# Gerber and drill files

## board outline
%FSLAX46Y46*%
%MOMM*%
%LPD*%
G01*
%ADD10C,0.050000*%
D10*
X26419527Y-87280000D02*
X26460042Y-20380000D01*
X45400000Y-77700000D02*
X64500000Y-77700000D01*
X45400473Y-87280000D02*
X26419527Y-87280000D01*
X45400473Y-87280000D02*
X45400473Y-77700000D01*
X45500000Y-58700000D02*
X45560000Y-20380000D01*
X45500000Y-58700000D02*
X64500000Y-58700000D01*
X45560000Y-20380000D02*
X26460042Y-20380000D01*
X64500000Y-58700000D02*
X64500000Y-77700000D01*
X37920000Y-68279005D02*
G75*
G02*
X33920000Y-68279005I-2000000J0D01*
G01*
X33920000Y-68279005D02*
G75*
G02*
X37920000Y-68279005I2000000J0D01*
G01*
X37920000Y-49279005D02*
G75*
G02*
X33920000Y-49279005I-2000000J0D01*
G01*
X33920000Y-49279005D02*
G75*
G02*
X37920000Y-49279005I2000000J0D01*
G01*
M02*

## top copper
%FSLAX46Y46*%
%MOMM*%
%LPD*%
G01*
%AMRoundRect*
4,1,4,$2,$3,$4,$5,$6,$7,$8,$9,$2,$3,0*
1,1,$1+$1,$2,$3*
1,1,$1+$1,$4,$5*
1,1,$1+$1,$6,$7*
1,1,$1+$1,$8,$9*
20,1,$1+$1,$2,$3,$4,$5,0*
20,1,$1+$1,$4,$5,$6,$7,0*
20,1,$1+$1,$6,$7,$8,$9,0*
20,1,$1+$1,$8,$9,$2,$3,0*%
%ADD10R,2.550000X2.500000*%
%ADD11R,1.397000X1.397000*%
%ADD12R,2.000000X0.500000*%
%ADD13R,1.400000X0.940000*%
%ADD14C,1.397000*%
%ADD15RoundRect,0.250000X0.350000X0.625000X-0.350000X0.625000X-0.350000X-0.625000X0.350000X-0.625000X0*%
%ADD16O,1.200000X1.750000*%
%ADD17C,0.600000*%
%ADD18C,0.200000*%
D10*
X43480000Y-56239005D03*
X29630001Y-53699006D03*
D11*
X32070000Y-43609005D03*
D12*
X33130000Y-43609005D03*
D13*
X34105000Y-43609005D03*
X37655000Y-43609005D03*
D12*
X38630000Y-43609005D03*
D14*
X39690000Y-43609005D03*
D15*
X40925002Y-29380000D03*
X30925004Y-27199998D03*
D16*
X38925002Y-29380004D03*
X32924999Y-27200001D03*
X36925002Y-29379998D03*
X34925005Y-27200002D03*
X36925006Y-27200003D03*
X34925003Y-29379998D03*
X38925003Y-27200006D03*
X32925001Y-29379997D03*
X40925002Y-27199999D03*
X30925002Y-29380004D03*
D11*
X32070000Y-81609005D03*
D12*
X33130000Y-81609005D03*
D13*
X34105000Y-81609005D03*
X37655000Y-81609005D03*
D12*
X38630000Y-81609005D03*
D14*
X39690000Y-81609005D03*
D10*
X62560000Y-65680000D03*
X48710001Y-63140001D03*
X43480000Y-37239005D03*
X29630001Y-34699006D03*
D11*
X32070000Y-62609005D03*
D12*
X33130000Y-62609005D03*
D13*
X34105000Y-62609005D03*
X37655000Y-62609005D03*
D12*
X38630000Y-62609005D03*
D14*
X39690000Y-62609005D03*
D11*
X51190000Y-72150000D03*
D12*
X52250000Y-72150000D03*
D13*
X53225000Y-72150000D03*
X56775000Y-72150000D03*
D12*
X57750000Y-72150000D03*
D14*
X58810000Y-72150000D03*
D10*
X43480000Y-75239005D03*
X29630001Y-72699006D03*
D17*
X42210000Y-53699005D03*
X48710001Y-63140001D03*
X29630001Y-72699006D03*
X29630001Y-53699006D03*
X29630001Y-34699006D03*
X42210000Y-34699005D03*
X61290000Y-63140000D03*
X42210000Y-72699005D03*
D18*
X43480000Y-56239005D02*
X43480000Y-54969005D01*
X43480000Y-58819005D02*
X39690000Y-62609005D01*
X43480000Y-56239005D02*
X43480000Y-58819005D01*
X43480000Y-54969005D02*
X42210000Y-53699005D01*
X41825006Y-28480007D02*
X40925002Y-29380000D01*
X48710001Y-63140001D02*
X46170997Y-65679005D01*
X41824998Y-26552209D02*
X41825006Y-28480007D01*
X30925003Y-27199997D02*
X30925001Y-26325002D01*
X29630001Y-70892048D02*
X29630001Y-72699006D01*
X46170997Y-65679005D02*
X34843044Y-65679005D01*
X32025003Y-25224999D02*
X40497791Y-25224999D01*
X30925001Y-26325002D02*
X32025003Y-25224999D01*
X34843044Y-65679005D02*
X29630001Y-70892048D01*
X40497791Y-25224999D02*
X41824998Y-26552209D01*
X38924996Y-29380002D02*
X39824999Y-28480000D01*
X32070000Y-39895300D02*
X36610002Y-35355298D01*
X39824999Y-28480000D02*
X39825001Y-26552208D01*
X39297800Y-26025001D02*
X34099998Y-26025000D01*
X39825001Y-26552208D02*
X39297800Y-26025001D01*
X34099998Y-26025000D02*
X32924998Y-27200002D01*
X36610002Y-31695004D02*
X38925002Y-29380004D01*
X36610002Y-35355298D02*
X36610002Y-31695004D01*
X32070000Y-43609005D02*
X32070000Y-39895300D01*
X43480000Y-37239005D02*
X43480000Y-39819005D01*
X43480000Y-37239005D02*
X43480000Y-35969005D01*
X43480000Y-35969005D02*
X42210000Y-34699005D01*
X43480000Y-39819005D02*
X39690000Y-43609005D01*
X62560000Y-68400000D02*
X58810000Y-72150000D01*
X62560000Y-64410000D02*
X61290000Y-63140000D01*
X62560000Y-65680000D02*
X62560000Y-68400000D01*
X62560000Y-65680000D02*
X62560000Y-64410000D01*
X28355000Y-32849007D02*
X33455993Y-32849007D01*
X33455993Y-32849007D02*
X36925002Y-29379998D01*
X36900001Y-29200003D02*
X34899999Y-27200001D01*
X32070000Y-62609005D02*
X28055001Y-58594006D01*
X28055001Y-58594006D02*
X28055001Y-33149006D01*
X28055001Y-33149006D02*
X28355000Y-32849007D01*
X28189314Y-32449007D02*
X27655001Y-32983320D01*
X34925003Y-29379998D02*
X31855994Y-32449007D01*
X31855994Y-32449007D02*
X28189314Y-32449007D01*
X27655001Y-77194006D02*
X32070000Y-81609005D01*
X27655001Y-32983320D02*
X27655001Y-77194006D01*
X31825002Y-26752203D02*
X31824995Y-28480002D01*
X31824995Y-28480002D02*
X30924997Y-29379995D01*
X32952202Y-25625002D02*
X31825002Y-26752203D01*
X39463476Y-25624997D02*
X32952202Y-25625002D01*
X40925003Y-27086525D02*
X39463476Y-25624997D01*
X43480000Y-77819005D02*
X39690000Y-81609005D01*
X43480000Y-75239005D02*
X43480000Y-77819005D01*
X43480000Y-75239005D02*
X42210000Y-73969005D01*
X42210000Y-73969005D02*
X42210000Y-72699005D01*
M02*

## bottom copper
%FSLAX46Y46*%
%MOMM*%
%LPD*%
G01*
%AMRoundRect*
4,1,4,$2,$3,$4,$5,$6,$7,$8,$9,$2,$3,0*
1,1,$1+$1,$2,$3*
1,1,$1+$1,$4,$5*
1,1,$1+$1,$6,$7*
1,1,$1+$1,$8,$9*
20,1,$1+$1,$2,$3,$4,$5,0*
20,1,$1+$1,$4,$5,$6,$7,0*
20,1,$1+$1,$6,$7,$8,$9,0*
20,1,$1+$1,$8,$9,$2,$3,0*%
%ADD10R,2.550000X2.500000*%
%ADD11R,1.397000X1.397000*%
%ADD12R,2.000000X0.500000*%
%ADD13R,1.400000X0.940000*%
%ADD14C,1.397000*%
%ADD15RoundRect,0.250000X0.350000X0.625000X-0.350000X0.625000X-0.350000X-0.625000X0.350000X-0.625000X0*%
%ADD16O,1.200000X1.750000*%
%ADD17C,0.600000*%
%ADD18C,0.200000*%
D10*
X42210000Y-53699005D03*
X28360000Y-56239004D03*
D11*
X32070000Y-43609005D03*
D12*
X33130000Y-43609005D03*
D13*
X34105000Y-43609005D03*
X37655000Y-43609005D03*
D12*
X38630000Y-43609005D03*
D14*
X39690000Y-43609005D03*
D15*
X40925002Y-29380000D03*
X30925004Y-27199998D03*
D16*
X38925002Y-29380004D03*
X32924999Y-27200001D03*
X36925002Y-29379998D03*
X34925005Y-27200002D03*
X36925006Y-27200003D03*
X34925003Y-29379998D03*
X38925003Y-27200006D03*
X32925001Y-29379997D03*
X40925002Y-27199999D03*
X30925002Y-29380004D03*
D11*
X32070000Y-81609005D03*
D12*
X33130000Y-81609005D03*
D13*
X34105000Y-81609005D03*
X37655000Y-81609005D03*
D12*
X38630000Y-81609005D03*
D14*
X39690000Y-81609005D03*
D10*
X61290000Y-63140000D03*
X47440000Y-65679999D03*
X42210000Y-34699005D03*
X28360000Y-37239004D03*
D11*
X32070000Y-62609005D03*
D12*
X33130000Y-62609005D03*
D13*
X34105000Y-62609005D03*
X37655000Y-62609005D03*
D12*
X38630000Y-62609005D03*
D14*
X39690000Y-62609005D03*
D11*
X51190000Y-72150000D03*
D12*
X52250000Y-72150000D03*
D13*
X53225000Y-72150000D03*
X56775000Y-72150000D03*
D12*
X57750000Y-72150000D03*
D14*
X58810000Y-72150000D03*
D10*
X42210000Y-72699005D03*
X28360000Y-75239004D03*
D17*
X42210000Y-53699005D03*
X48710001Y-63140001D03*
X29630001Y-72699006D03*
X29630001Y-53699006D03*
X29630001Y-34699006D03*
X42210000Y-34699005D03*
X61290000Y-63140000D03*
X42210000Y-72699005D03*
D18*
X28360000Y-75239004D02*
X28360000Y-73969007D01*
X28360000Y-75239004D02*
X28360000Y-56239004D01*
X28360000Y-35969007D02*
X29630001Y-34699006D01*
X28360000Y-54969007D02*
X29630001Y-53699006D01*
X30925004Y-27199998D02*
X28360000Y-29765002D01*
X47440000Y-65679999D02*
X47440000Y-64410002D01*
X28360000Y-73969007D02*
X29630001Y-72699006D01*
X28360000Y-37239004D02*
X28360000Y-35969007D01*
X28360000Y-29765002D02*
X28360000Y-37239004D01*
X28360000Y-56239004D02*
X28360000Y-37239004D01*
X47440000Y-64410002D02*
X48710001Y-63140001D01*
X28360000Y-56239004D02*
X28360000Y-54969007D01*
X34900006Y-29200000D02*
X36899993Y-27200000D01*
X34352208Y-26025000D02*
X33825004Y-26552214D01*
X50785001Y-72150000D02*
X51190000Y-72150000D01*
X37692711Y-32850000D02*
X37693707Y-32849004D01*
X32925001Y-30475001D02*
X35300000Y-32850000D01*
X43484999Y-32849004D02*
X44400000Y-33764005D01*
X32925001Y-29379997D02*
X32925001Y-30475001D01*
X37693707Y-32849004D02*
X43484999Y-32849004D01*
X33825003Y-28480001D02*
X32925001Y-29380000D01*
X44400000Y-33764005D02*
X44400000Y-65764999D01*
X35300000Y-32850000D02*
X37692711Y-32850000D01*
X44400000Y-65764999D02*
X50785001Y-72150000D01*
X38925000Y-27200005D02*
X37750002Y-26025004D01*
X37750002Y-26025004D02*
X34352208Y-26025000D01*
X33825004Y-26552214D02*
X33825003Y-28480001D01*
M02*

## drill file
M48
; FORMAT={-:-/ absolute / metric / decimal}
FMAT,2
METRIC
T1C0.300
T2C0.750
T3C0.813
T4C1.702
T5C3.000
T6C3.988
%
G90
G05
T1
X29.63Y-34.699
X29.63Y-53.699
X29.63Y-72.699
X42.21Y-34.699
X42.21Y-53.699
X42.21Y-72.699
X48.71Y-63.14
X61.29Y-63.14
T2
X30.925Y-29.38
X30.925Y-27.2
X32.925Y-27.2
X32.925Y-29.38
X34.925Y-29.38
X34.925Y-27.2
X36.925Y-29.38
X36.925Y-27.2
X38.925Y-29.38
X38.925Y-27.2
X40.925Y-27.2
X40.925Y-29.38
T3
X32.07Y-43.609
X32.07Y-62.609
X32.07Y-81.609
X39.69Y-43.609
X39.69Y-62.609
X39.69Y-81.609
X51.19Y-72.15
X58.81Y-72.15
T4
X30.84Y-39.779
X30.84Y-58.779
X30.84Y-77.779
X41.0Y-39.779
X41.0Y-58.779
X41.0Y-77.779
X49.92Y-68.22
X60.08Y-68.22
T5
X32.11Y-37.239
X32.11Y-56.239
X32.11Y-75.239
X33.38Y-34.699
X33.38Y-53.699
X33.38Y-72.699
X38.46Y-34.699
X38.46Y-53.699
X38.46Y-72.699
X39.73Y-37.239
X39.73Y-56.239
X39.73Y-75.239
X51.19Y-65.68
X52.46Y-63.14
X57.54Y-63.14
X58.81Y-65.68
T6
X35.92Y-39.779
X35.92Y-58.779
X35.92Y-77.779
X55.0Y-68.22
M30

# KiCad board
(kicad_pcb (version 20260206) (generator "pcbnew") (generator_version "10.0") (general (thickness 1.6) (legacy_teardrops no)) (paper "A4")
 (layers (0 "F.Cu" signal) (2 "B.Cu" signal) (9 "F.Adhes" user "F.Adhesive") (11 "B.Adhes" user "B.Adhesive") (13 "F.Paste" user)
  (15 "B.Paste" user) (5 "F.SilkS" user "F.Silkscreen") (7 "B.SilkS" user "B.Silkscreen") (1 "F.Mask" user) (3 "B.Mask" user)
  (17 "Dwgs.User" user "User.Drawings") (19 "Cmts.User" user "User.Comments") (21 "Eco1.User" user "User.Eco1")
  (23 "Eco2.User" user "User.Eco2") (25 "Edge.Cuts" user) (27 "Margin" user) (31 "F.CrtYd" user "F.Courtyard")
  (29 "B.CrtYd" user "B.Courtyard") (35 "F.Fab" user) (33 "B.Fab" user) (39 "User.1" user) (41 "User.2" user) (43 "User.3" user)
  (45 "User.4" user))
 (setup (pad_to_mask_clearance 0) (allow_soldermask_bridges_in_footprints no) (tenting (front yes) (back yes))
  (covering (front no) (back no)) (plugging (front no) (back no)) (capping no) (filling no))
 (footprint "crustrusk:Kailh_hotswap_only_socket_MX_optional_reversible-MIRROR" (layer "F.Cu") (at 35.92 58.779005)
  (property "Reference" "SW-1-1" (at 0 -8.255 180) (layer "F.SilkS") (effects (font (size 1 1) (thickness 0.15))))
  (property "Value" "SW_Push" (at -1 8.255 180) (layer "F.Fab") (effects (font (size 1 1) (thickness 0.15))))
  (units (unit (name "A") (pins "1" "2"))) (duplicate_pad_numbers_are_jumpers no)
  (pad "" np_thru_hole circle (at -5.08 0) (size 1.7018 1.7018) (drill 1.7018) (layers "*.Cu" "*.Mask"))
  (pad "" np_thru_hole circle (at -3.81 -2.54 180) (size 3 3) (drill 3) (layers "*.Cu" "*.Mask"))
  (pad "" np_thru_hole circle (at -2.54 -5.079998) (size 3 3) (drill 3) (layers "*.Cu" "*.Mask"))
  (pad "" np_thru_hole circle (at 0 0) (size 3.9878 3.9878) (drill 3.9878) (layers "*.Cu" "*.Mask"))
  (pad "" np_thru_hole circle (at 2.540002 -5.080001 180) (size 3 3) (drill 3) (layers "*.Cu" "*.Mask"))
  (pad "" np_thru_hole circle (at 3.81 -2.54) (size 3 3) (drill 3) (layers "*.Cu" "*.Mask"))
  (pad "" np_thru_hole circle (at 5.08 0) (size 1.7018 1.7018) (drill 1.7018) (layers "*.Cu" "*.Mask"))
  (pad "1" smd rect (at 6.29 -5.08 180) (size 2.55 2.5) (layers "B.Cu" "B.Mask" "B.Paste") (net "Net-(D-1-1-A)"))
  (pad "1" smd rect (at 7.56 -2.54) (size 2.55 2.5) (layers "F.Cu" "F.Mask" "F.Paste") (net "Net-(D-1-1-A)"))
  (pad "2" smd rect (at -7.56 -2.540001 180) (size 2.55 2.5) (layers "B.Cu" "B.Mask" "B.Paste") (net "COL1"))
  (pad "2" smd rect (at -6.289999 -5.079999) (size 2.55 2.5) (layers "F.Cu" "F.Mask" "F.Paste") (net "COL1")))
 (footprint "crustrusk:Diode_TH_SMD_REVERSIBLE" (layer "F.Cu") (at 35.88 43.609005)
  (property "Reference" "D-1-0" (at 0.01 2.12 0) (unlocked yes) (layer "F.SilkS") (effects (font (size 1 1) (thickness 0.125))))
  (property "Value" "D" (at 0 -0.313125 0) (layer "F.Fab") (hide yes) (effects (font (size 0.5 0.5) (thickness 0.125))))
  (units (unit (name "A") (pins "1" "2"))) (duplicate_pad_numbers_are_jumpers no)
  (pad "1" thru_hole rect (at -3.81 0) (size 1.397 1.397) (drill 0.8128) (layers "*.Cu" "*.Mask") (remove_unused_layers no) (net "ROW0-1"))
  (pad "1" smd rect (at -2.75 0 180) (size 2 0.5) (layers "F.Cu") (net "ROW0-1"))
  (pad "1" smd rect (at -2.75 0) (size 2 0.5) (layers "B.Cu") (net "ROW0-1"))
  (pad "1" smd rect (at -1.775 0 180) (size 1.4 0.94) (layers "F.Cu" "F.Mask" "F.Paste") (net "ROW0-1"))
  (pad "1" smd rect (at -1.775 0) (size 1.4 0.94) (layers "B.Cu" "B.Mask" "B.Paste") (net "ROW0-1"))
  (pad "2" smd rect (at 1.775 0 180) (size 1.4 0.94) (layers "F.Cu" "F.Mask" "F.Paste") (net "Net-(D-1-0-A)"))
  (pad "2" smd rect (at 1.775 0) (size 1.4 0.94) (layers "B.Cu" "B.Mask" "B.Paste") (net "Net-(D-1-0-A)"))
  (pad "2" smd rect (at 2.75 0 180) (size 2 0.5) (layers "F.Cu") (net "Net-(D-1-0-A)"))
  (pad "2" smd rect (at 2.75 0) (size 2 0.5) (layers "B.Cu") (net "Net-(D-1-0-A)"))
  (pad "2" thru_hole circle (at 3.81 0) (size 1.397 1.397) (drill 0.8128) (layers "*.Cu" "*.Mask") (remove_unused_layers no)
   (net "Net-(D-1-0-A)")))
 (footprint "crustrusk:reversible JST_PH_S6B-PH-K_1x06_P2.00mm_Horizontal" (layer "F.Cu") (at 40.925002 29.38 180)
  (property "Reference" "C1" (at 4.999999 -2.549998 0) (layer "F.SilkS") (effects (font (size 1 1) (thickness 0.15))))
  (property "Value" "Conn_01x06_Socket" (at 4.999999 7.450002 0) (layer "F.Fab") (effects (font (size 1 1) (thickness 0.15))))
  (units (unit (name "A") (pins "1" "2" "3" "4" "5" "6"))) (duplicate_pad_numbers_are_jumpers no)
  (pad "1" thru_hole roundrect (at 0 0 180) (size 1.2 1.75) (drill 0.75) (layers "*.Cu" "*.Mask") (remove_unused_layers no)
   (roundrect_rratio 0.208333) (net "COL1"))
  (pad "1" thru_hole roundrect (at 9.999998 2.180002 180) (size 1.2 1.75) (drill 0.75) (layers "*.Cu" "*.Mask") (remove_unused_layers no)
   (roundrect_rratio 0.208333) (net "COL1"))
  (pad "2" thru_hole oval (at 2 -0.000004 180) (size 1.2 1.75) (drill 0.75) (layers "*.Cu" "*.Mask") (remove_unused_layers no)
   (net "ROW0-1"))
  (pad "2" thru_hole oval (at 8.000003 2.179999 180) (size 1.2 1.75) (drill 0.75) (layers "*.Cu" "*.Mask") (remove_unused_layers no)
   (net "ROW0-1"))
  (pad "3" thru_hole oval (at 4 0.000002 180) (size 1.2 1.75) (drill 0.75) (layers "*.Cu" "*.Mask") (remove_unused_layers no) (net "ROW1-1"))
  (pad "3" thru_hole oval (at 5.999997 2.179998 180) (size 1.2 1.75) (drill 0.75) (layers "*.Cu" "*.Mask") (remove_unused_layers no)
   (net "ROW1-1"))
  (pad "4" thru_hole oval (at 3.999996 2.179997 180) (size 1.2 1.75) (drill 0.75) (layers "*.Cu" "*.Mask") (remove_unused_layers no)
   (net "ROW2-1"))
  (pad "4" thru_hole oval (at 5.999999 0.000002 180) (size 1.2 1.75) (drill 0.75) (layers "*.Cu" "*.Mask") (remove_unused_layers no)
   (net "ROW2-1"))
  (pad "5" thru_hole oval (at 1.999999 2.179994 180) (size 1.2 1.75) (drill 0.75) (layers "*.Cu" "*.Mask") (remove_unused_layers no)
   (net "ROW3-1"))
  (pad "5" thru_hole oval (at 8.000001 0.000003 180) (size 1.2 1.75) (drill 0.75) (layers "*.Cu" "*.Mask") (remove_unused_layers no)
   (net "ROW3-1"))
  (pad "6" thru_hole oval (at 0 2.180001 180) (size 1.2 1.75) (drill 0.75) (layers "*.Cu" "*.Mask") (remove_unused_layers no) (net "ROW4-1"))
  (pad "6" thru_hole oval (at 10 -0.000004 180) (size 1.2 1.75) (drill 0.75) (layers "*.Cu" "*.Mask") (remove_unused_layers no)
   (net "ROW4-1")))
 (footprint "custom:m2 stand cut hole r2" (layer "F.Cu") (at 35.92 68.279005)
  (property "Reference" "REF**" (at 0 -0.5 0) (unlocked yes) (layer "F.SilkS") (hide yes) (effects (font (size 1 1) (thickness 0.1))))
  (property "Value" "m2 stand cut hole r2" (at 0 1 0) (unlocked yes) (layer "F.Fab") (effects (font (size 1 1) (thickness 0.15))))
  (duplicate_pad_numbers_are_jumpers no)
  (fp_circle (center 0 0) (end 2 0) (stroke (width 0.05) (type default)) (fill no) (layer "Edge.Cuts")))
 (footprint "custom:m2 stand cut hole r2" (layer "F.Cu") (at 35.92 49.279005)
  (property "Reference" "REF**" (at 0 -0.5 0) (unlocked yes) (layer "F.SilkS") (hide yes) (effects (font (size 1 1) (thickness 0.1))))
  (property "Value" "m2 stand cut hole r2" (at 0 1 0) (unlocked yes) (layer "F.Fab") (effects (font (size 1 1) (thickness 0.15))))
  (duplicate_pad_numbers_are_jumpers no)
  (fp_circle (center 0 0) (end 2 0) (stroke (width 0.05) (type default)) (fill no) (layer "Edge.Cuts")))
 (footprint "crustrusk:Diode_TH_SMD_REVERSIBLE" (layer "F.Cu") (at 35.88 81.609005)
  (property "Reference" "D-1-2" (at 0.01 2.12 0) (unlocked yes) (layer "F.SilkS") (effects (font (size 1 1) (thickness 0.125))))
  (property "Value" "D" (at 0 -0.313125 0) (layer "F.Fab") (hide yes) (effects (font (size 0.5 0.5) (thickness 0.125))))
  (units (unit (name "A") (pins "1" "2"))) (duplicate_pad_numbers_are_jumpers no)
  (pad "1" thru_hole rect (at -3.81 0) (size 1.397 1.397) (drill 0.8128) (layers "*.Cu" "*.Mask") (remove_unused_layers no) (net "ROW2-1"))
  (pad "1" smd rect (at -2.75 0 180) (size 2 0.5) (layers "F.Cu") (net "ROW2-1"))
  (pad "1" smd rect (at -2.75 0) (size 2 0.5) (layers "B.Cu") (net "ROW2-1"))
  (pad "1" smd rect (at -1.775 0 180) (size 1.4 0.94) (layers "F.Cu" "F.Mask" "F.Paste") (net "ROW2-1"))
  (pad "1" smd rect (at -1.775 0) (size 1.4 0.94) (layers "B.Cu" "B.Mask" "B.Paste") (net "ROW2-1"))
  (pad "2" smd rect (at 1.775 0 180) (size 1.4 0.94) (layers "F.Cu" "F.Mask" "F.Paste") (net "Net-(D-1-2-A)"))
  (pad "2" smd rect (at 1.775 0) (size 1.4 0.94) (layers "B.Cu" "B.Mask" "B.Paste") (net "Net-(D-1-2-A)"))
  (pad "2" smd rect (at 2.75 0 180) (size 2 0.5) (layers "F.Cu") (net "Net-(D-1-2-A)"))
  (pad "2" smd rect (at 2.75 0) (size 2 0.5) (layers "B.Cu") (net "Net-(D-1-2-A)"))
  (pad "2" thru_hole circle (at 3.81 0) (size 1.397 1.397) (drill 0.8128) (layers "*.Cu" "*.Mask") (remove_unused_layers no)
   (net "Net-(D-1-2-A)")))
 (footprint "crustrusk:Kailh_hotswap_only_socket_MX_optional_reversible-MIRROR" (layer "F.Cu") (at 55 68.22)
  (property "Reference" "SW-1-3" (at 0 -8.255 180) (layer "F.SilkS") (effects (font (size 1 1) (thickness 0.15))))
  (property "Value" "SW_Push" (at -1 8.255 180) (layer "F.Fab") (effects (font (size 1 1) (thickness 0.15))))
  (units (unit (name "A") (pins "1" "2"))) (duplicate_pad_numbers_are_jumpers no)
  (pad "" np_thru_hole circle (at -5.08 0) (size 1.7018 1.7018) (drill 1.7018) (layers "*.Cu" "*.Mask"))
  (pad "" np_thru_hole circle (at -3.81 -2.54 180) (size 3 3) (drill 3) (layers "*.Cu" "*.Mask"))
  (pad "" np_thru_hole circle (at -2.54 -5.079998) (size 3 3) (drill 3) (layers "*.Cu" "*.Mask"))
  (pad "" np_thru_hole circle (at 0 0) (size 3.9878 3.9878) (drill 3.9878) (layers "*.Cu" "*.Mask"))
  (pad "" np_thru_hole circle (at 2.540002 -5.080001 180) (size 3 3) (drill 3) (layers "*.Cu" "*.Mask"))
  (pad "" np_thru_hole circle (at 3.81 -2.54) (size 3 3) (drill 3) (layers "*.Cu" "*.Mask"))
  (pad "" np_thru_hole circle (at 5.08 0) (size 1.7018 1.7018) (drill 1.7018) (layers "*.Cu" "*.Mask"))
  (pad "1" smd rect (at 6.29 -5.08 180) (size 2.55 2.5) (layers "B.Cu" "B.Mask" "B.Paste") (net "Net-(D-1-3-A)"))
  (pad "1" smd rect (at 7.56 -2.54) (size 2.55 2.5) (layers "F.Cu" "F.Mask" "F.Paste") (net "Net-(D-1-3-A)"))
  (pad "2" smd rect (at -7.56 -2.540001 180) (size 2.55 2.5) (layers "B.Cu" "B.Mask" "B.Paste") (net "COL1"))
  (pad "2" smd rect (at -6.289999 -5.079999) (size 2.55 2.5) (layers "F.Cu" "F.Mask" "F.Paste") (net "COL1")))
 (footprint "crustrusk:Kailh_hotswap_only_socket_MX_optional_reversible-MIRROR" (layer "F.Cu") (at 35.92 39.779005)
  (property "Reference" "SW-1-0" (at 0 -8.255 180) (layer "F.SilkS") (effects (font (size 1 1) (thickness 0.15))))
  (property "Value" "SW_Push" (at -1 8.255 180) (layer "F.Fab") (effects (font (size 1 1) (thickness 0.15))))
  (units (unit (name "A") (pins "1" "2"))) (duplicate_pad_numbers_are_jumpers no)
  (pad "" np_thru_hole circle (at -5.08 0) (size 1.7018 1.7018) (drill 1.7018) (layers "*.Cu" "*.Mask"))
  (pad "" np_thru_hole circle (at -3.81 -2.54 180) (size 3 3) (drill 3) (layers "*.Cu" "*.Mask"))
  (pad "" np_thru_hole circle (at -2.54 -5.079998) (size 3 3) (drill 3) (layers "*.Cu" "*.Mask"))
  (pad "" np_thru_hole circle (at 0 0) (size 3.9878 3.9878) (drill 3.9878) (layers "*.Cu" "*.Mask"))
  (pad "" np_thru_hole circle (at 2.540002 -5.080001 180) (size 3 3) (drill 3) (layers "*.Cu" "*.Mask"))
  (pad "" np_thru_hole circle (at 3.81 -2.54) (size 3 3) (drill 3) (layers "*.Cu" "*.Mask"))
  (pad "" np_thru_hole circle (at 5.08 0) (size 1.7018 1.7018) (drill 1.7018) (layers "*.Cu" "*.Mask"))
  (pad "1" smd rect (at 6.29 -5.08 180) (size 2.55 2.5) (layers "B.Cu" "B.Mask" "B.Paste") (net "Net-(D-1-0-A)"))
  (pad "1" smd rect (at 7.56 -2.54) (size 2.55 2.5) (layers "F.Cu" "F.Mask" "F.Paste") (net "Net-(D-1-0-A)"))
  (pad "2" smd rect (at -7.56 -2.540001 180) (size 2.55 2.5) (layers "B.Cu" "B.Mask" "B.Paste") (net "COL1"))
  (pad "2" smd rect (at -6.289999 -5.079999) (size 2.55 2.5) (layers "F.Cu" "F.Mask" "F.Paste") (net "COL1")))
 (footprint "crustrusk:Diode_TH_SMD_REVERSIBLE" (layer "F.Cu") (at 35.88 62.609005)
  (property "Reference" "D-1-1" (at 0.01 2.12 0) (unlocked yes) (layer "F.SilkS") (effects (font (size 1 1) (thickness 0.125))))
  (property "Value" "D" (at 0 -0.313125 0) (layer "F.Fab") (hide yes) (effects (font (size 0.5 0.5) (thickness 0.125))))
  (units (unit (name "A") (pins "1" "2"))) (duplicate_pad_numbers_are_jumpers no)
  (pad "1" thru_hole rect (at -3.81 0) (size 1.397 1.397) (drill 0.8128) (layers "*.Cu" "*.Mask") (remove_unused_layers no) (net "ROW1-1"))
  (pad "1" smd rect (at -2.75 0 180) (size 2 0.5) (layers "F.Cu") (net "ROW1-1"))
  (pad "1" smd rect (at -2.75 0) (size 2 0.5) (layers "B.Cu") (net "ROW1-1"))
  (pad "1" smd rect (at -1.775 0 180) (size 1.4 0.94) (layers "F.Cu" "F.Mask" "F.Paste") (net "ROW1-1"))
  (pad "1" smd rect (at -1.775 0) (size 1.4 0.94) (layers "B.Cu" "B.Mask" "B.Paste") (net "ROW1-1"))
  (pad "2" smd rect (at 1.775 0 180) (size 1.4 0.94) (layers "F.Cu" "F.Mask" "F.Paste") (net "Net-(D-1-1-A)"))
  (pad "2" smd rect (at 1.775 0) (size 1.4 0.94) (layers "B.Cu" "B.Mask" "B.Paste") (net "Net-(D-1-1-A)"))
  (pad "2" smd rect (at 2.75 0 180) (size 2 0.5) (layers "F.Cu") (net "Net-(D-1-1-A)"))
  (pad "2" smd rect (at 2.75 0) (size 2 0.5) (layers "B.Cu") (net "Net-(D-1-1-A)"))
  (pad "2" thru_hole circle (at 3.81 0) (size 1.397 1.397) (drill 0.8128) (layers "*.Cu" "*.Mask") (remove_unused_layers no)
   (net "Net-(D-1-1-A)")))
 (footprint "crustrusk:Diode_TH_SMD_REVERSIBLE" (layer "F.Cu") (at 55 72.15)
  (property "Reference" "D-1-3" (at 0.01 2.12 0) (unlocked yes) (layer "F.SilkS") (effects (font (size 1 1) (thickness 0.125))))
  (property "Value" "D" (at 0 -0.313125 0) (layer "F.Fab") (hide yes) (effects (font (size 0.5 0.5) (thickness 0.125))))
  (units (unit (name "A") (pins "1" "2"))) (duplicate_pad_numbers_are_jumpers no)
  (pad "1" thru_hole rect (at -3.81 0) (size 1.397 1.397) (drill 0.8128) (layers "*.Cu" "*.Mask") (remove_unused_layers no) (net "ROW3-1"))
  (pad "1" smd rect (at -2.75 0 180) (size 2 0.5) (layers "F.Cu") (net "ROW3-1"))
  (pad "1" smd rect (at -2.75 0) (size 2 0.5) (layers "B.Cu") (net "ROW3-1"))
  (pad "1" smd rect (at -1.775 0 180) (size 1.4 0.94) (layers "F.Cu" "F.Mask" "F.Paste") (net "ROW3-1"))
  (pad "1" smd rect (at -1.775 0) (size 1.4 0.94) (layers "B.Cu" "B.Mask" "B.Paste") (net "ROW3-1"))
  (pad "2" smd rect (at 1.775 0 180) (size 1.4 0.94) (layers "F.Cu" "F.Mask" "F.Paste") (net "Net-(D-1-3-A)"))
  (pad "2" smd rect (at 1.775 0) (size 1.4 0.94) (layers "B.Cu" "B.Mask" "B.Paste") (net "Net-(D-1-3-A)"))
  (pad "2" smd rect (at 2.75 0 180) (size 2 0.5) (layers "F.Cu") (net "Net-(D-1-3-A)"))
  (pad "2" smd rect (at 2.75 0) (size 2 0.5) (layers "B.Cu") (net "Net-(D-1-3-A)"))
  (pad "2" thru_hole circle (at 3.81 0) (size 1.397 1.397) (drill 0.8128) (layers "*.Cu" "*.Mask") (remove_unused_layers no)
   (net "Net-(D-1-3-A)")))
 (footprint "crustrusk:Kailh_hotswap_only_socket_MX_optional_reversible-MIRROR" (layer "F.Cu") (at 35.92 77.779005)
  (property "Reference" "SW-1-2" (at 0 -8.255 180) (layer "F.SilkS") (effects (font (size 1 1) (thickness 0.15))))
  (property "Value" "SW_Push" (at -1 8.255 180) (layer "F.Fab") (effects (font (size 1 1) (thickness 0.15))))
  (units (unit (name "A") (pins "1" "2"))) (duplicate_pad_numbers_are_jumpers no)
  (pad "" np_thru_hole circle (at -5.08 0) (size 1.7018 1.7018) (drill 1.7018) (layers "*.Cu" "*.Mask"))
  (pad "" np_thru_hole circle (at -3.81 -2.54 180) (size 3 3) (drill 3) (layers "*.Cu" "*.Mask"))
  (pad "" np_thru_hole circle (at -2.54 -5.079998) (size 3 3) (drill 3) (layers "*.Cu" "*.Mask"))
  (pad "" np_thru_hole circle (at 0 0) (size 3.9878 3.9878) (drill 3.9878) (layers "*.Cu" "*.Mask"))
  (pad "" np_thru_hole circle (at 2.540002 -5.080001 180) (size 3 3) (drill 3) (layers "*.Cu" "*.Mask"))
  (pad "" np_thru_hole circle (at 3.81 -2.54) (size 3 3) (drill 3) (layers "*.Cu" "*.Mask"))
  (pad "" np_thru_hole circle (at 5.08 0) (size 1.7018 1.7018) (drill 1.7018) (layers "*.Cu" "*.Mask"))
  (pad "1" smd rect (at 6.29 -5.08 180) (size 2.55 2.5) (layers "B.Cu" "B.Mask" "B.Paste") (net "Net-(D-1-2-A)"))
  (pad "1" smd rect (at 7.56 -2.54) (size 2.55 2.5) (layers "F.Cu" "F.Mask" "F.Paste") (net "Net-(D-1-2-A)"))
  (pad "2" smd rect (at -7.56 -2.540001 180) (size 2.55 2.5) (layers "B.Cu" "B.Mask" "B.Paste") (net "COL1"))
  (pad "2" smd rect (at -6.289999 -5.079999) (size 2.55 2.5) (layers "F.Cu" "F.Mask" "F.Paste") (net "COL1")))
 (gr_line (start 26.419527 87.28) (end 26.460042 20.38) (stroke (width 0.05) (type default)) (layer "Edge.Cuts"))
 (gr_line (start 45.4 77.7) (end 64.5 77.7) (stroke (width 0.05) (type default)) (layer "Edge.Cuts"))
 (gr_line (start 45.400473 87.28) (end 26.419527 87.28) (stroke (width 0.05) (type default)) (layer "Edge.Cuts"))
 (gr_line (start 45.400473 87.28) (end 45.400473 77.7) (stroke (width 0.05) (type default)) (layer "Edge.Cuts"))
 (gr_line (start 45.5 58.7) (end 45.56 20.38) (stroke (width 0.05) (type default)) (layer "Edge.Cuts"))
 (gr_line (start 45.5 58.7) (end 64.5 58.7) (stroke (width 0.05) (type default)) (layer "Edge.Cuts"))
 (gr_line (start 45.56 20.38) (end 26.460042 20.38) (stroke (width 0.05) (type default)) (layer "Edge.Cuts"))
 (gr_line (start 64.5 58.7) (end 64.5 77.7) (stroke (width 0.05) (type default)) (layer "Edge.Cuts"))
 (segment (start 43.48 56.239005) (end 43.48 54.969005) (width 0.2) (layer "F.Cu") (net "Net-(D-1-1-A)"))
 (segment (start 43.48 58.819005) (end 39.69 62.609005) (width 0.2) (layer "F.Cu") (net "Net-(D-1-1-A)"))
 (segment (start 43.48 56.239005) (end 43.48 58.819005) (width 0.2) (layer "F.Cu") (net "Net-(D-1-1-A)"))
 (segment (start 43.48 54.969005) (end 42.21 53.699005) (width 0.2) (layer "F.Cu") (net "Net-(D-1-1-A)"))
 (via (at 42.21 53.699005) (size 0.6) (drill 0.3) (layers "F.Cu" "B.Cu") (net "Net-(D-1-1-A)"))
 (segment (start 41.825006 28.480007) (end 40.925002 29.38) (width 0.2) (layer "F.Cu") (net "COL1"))
 (segment (start 48.710001 63.140001) (end 46.170997 65.679005) (width 0.2) (layer "F.Cu") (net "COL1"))
 (segment (start 41.824998 26.552209) (end 41.825006 28.480007) (width 0.2) (layer "F.Cu") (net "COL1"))
 (segment (start 30.925003 27.199997) (end 30.925001 26.325002) (width 0.2) (layer "F.Cu") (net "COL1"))
 (segment (start 29.630001 70.892048) (end 29.630001 72.699006) (width 0.2) (layer "F.Cu") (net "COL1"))
 (segment (start 46.170997 65.679005) (end 34.843044 65.679005) (width 0.2) (layer "F.Cu") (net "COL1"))
 (segment (start 32.025003 25.224999) (end 40.497791 25.224999) (width 0.2) (layer "F.Cu") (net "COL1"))
 (segment (start 30.925001 26.325002) (end 32.025003 25.224999) (width 0.2) (layer "F.Cu") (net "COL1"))
 (segment (start 34.843044 65.679005) (end 29.630001 70.892048) (width 0.2) (layer "F.Cu") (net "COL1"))
 (segment (start 40.497791 25.224999) (end 41.824998 26.552209) (width 0.2) (layer "F.Cu") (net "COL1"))
 (via (at 48.710001 63.140001) (size 0.6) (drill 0.3) (layers "F.Cu" "B.Cu") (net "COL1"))
 (via (at 29.630001 72.699006) (size 0.6) (drill 0.3) (layers "F.Cu" "B.Cu") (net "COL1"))
 (via (at 29.630001 53.699006) (size 0.6) (drill 0.3) (layers "F.Cu" "B.Cu") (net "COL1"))
 (via (at 29.630001 34.699006) (size 0.6) (drill 0.3) (layers "F.Cu" "B.Cu") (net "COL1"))
 (segment (start 28.36 75.239004) (end 28.36 73.969007) (width 0.2) (layer "B.Cu") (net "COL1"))
 (segment (start 28.36 75.239004) (end 28.36 56.239004) (width 0.2) (layer "B.Cu") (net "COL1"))
 (segment (start 28.36 35.969007) (end 29.630001 34.699006) (width 0.2) (layer "B.Cu") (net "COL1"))
 (segment (start 28.36 54.969007) (end 29.630001 53.699006) (width 0.2) (layer "B.Cu") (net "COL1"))
 (segment (start 30.925004 27.199998) (end 28.36 29.765002) (width 0.2) (layer "B.Cu") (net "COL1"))
 (segment (start 47.44 65.679999) (end 47.44 64.410002) (width 0.2) (layer "B.Cu") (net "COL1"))
 (segment (start 28.36 73.969007) (end 29.630001 72.699006) (width 0.2) (layer "B.Cu") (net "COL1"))
 (segment (start 28.36 37.239004) (end 28.36 35.969007) (width 0.2) (layer "B.Cu") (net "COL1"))
 (segment (start 28.36 29.765002) (end 28.36 37.239004) (width 0.2) (layer "B.Cu") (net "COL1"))
 (segment (start 28.36 56.239004) (end 28.36 37.239004) (width 0.2) (layer "B.Cu") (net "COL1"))
 (segment (start 47.44 64.410002) (end 48.710001 63.140001) (width 0.2) (layer "B.Cu") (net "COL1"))
 (segment (start 28.36 56.239004) (end 28.36 54.969007) (width 0.2) (layer "B.Cu") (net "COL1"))
 (segment (start 38.924996 29.380002) (end 39.824999 28.48) (width 0.2) (layer "F.Cu") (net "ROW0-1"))
 (segment (start 32.07 39.8953) (end 36.610002 35.355298) (width 0.2) (layer "F.Cu") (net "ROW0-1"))
 (segment (start 39.824999 28.48) (end 39.825001 26.552208) (width 0.2) (layer "F.Cu") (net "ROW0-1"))
 (segment (start 39.2978 26.025001) (end 34.099998 26.025) (width 0.2) (layer "F.Cu") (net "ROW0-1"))
 (segment (start 39.825001 26.552208) (end 39.2978 26.025001) (width 0.2) (layer "F.Cu") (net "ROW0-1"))
 (segment (start 34.099998 26.025) (end 32.924998 27.200002) (width 0.2) (layer "F.Cu") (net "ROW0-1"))
 (segment (start 36.610002 31.695004) (end 38.925002 29.380004) (width 0.2) (layer "F.Cu") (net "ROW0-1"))
 (segment (start 36.610002 35.355298) (end 36.610002 31.695004) (width 0.2) (layer "F.Cu") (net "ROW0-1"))
 (segment (start 32.07 43.609005) (end 32.07 39.8953) (width 0.2) (layer "F.Cu") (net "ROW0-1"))
 (segment (start 43.48 37.239005) (end 43.48 39.819005) (width 0.2) (layer "F.Cu") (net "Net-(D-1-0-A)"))
 (segment (start 43.48 37.239005) (end 43.48 35.969005) (width 0.2) (layer "F.Cu") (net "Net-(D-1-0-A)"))
 (segment (start 43.48 35.969005) (end 42.21 34.699005) (width 0.2) (layer "F.Cu") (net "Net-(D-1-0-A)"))
 (segment (start 43.48 39.819005) (end 39.69 43.609005) (width 0.2) (layer "F.Cu") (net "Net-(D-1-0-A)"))
 (via (at 42.21 34.699005) (size 0.6) (drill 0.3) (layers "F.Cu" "B.Cu") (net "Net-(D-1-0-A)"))
 (segment (start 62.56 68.4) (end 58.81 72.15) (width 0.2) (layer "F.Cu") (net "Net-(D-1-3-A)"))
 (segment (start 62.56 64.41) (end 61.29 63.14) (width 0.2) (layer "F.Cu") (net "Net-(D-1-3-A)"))
 (segment (start 62.56 65.68) (end 62.56 68.4) (width 0.2) (layer "F.Cu") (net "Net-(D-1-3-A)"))
 (segment (start 62.56 65.68) (end 62.56 64.41) (width 0.2) (layer "F.Cu") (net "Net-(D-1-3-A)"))
 (via (at 61.29 63.14) (size 0.6) (drill 0.3) (layers "F.Cu" "B.Cu") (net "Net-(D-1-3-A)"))
 (segment (start 28.355 32.849007) (end 33.455993 32.849007) (width 0.2) (layer "F.Cu") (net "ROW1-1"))
 (segment (start 33.455993 32.849007) (end 36.925002 29.379998) (width 0.2) (layer "F.Cu") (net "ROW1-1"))
 (segment (start 36.900001 29.200003) (end 34.899999 27.200001) (width 0.2) (layer "F.Cu") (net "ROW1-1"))
 (segment (start 32.07 62.609005) (end 28.055001 58.594006) (width 0.2) (layer "F.Cu") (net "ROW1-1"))
 (segment (start 28.055001 58.594006) (end 28.055001 33.149006) (width 0.2) (layer "F.Cu") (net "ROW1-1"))
 (segment (start 28.055001 33.149006) (end 28.355 32.849007) (width 0.2) (layer "F.Cu") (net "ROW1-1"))
 (segment (start 28.189314 32.449007) (end 27.655001 32.98332) (width 0.2) (layer "F.Cu") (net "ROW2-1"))
 (segment (start 34.925003 29.379998) (end 31.855994 32.449007) (width 0.2) (layer "F.Cu") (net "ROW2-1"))
 (segment (start 31.855994 32.449007) (end 28.189314 32.449007) (width 0.2) (layer "F.Cu") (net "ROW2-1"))
 (segment (start 27.655001 77.194006) (end 32.07 81.609005) (width 0.2) (layer "F.Cu") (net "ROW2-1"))
 (segment (start 27.655001 32.98332) (end 27.655001 77.194006) (width 0.2) (layer "F.Cu") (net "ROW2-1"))
 (segment (start 34.900006 29.2) (end 36.899993 27.2) (width 0.2) (layer "B.Cu") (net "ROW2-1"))
 (segment (start 34.352208 26.025) (end 33.825004 26.552214) (width 0.2) (layer "B.Cu") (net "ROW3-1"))
 (segment (start 50.785001 72.15) (end 51.19 72.15) (width 0.2) (layer "B.Cu") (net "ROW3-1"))
 (segment (start 37.692711 32.85) (end 37.693707 32.849004) (width 0.2) (layer "B.Cu") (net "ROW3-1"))
 (segment (start 32.925001 30.475001) (end 35.3 32.85) (width 0.2) (layer "B.Cu") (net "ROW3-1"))
 (segment (start 43.484999 32.849004) (end 44.4 33.764005) (width 0.2) (layer "B.Cu") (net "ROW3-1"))
 (segment (start 32.925001 29.379997) (end 32.925001 30.475001) (width 0.2) (layer "B.Cu") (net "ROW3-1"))
 (segment (start 37.693707 32.849004) (end 43.484999 32.849004) (width 0.2) (layer "B.Cu") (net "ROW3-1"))
 (segment (start 33.825003 28.480001) (end 32.925001 29.38) (width 0.2) (layer "B.Cu") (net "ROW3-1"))
 (segment (start 44.4 33.764005) (end 44.4 65.764999) (width 0.2) (layer "B.Cu") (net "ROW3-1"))
 (segment (start 35.3 32.85) (end 37.692711 32.85) (width 0.2) (layer "B.Cu") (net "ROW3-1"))
 (segment (start 44.4 65.764999) (end 50.785001 72.15) (width 0.2) (layer "B.Cu") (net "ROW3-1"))
 (segment (start 38.925 27.200005) (end 37.750002 26.025004) (width 0.2) (layer "B.Cu") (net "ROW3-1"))
 (segment (start 37.750002 26.025004) (end 34.352208 26.025) (width 0.2) (layer "B.Cu") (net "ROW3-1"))
 (segment (start 33.825004 26.552214) (end 33.825003 28.480001) (width 0.2) (layer "B.Cu") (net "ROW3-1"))
 (segment (start 31.825002 26.752203) (end 31.824995 28.480002) (width 0.2) (layer "F.Cu") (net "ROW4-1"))
 (segment (start 31.824995 28.480002) (end 30.924997 29.379995) (width 0.2) (layer "F.Cu") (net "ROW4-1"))
 (segment (start 32.952202 25.625002) (end 31.825002 26.752203) (width 0.2) (layer "F.Cu") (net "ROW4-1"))
 (segment (start 39.463476 25.624997) (end 32.952202 25.625002) (width 0.2) (layer "F.Cu") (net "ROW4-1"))
 (segment (start 40.925003 27.086525) (end 39.463476 25.624997) (width 0.2) (layer "F.Cu") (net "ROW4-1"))
 (segment (start 43.48 77.819005) (end 39.69 81.609005) (width 0.2) (layer "F.Cu") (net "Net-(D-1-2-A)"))
 (segment (start 43.48 75.239005) (end 43.48 77.819005) (width 0.2) (layer "F.Cu") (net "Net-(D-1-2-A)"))
 (segment (start 43.48 75.239005) (end 42.21 73.969005) (width 0.2) (layer "F.Cu") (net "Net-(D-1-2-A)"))
 (segment (start 42.21 73.969005) (end 42.21 72.699005) (width 0.2) (layer "F.Cu") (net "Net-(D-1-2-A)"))
 (via (at 42.21 72.699005) (size 0.6) (drill 0.3) (layers "F.Cu" "B.Cu") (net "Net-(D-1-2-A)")))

